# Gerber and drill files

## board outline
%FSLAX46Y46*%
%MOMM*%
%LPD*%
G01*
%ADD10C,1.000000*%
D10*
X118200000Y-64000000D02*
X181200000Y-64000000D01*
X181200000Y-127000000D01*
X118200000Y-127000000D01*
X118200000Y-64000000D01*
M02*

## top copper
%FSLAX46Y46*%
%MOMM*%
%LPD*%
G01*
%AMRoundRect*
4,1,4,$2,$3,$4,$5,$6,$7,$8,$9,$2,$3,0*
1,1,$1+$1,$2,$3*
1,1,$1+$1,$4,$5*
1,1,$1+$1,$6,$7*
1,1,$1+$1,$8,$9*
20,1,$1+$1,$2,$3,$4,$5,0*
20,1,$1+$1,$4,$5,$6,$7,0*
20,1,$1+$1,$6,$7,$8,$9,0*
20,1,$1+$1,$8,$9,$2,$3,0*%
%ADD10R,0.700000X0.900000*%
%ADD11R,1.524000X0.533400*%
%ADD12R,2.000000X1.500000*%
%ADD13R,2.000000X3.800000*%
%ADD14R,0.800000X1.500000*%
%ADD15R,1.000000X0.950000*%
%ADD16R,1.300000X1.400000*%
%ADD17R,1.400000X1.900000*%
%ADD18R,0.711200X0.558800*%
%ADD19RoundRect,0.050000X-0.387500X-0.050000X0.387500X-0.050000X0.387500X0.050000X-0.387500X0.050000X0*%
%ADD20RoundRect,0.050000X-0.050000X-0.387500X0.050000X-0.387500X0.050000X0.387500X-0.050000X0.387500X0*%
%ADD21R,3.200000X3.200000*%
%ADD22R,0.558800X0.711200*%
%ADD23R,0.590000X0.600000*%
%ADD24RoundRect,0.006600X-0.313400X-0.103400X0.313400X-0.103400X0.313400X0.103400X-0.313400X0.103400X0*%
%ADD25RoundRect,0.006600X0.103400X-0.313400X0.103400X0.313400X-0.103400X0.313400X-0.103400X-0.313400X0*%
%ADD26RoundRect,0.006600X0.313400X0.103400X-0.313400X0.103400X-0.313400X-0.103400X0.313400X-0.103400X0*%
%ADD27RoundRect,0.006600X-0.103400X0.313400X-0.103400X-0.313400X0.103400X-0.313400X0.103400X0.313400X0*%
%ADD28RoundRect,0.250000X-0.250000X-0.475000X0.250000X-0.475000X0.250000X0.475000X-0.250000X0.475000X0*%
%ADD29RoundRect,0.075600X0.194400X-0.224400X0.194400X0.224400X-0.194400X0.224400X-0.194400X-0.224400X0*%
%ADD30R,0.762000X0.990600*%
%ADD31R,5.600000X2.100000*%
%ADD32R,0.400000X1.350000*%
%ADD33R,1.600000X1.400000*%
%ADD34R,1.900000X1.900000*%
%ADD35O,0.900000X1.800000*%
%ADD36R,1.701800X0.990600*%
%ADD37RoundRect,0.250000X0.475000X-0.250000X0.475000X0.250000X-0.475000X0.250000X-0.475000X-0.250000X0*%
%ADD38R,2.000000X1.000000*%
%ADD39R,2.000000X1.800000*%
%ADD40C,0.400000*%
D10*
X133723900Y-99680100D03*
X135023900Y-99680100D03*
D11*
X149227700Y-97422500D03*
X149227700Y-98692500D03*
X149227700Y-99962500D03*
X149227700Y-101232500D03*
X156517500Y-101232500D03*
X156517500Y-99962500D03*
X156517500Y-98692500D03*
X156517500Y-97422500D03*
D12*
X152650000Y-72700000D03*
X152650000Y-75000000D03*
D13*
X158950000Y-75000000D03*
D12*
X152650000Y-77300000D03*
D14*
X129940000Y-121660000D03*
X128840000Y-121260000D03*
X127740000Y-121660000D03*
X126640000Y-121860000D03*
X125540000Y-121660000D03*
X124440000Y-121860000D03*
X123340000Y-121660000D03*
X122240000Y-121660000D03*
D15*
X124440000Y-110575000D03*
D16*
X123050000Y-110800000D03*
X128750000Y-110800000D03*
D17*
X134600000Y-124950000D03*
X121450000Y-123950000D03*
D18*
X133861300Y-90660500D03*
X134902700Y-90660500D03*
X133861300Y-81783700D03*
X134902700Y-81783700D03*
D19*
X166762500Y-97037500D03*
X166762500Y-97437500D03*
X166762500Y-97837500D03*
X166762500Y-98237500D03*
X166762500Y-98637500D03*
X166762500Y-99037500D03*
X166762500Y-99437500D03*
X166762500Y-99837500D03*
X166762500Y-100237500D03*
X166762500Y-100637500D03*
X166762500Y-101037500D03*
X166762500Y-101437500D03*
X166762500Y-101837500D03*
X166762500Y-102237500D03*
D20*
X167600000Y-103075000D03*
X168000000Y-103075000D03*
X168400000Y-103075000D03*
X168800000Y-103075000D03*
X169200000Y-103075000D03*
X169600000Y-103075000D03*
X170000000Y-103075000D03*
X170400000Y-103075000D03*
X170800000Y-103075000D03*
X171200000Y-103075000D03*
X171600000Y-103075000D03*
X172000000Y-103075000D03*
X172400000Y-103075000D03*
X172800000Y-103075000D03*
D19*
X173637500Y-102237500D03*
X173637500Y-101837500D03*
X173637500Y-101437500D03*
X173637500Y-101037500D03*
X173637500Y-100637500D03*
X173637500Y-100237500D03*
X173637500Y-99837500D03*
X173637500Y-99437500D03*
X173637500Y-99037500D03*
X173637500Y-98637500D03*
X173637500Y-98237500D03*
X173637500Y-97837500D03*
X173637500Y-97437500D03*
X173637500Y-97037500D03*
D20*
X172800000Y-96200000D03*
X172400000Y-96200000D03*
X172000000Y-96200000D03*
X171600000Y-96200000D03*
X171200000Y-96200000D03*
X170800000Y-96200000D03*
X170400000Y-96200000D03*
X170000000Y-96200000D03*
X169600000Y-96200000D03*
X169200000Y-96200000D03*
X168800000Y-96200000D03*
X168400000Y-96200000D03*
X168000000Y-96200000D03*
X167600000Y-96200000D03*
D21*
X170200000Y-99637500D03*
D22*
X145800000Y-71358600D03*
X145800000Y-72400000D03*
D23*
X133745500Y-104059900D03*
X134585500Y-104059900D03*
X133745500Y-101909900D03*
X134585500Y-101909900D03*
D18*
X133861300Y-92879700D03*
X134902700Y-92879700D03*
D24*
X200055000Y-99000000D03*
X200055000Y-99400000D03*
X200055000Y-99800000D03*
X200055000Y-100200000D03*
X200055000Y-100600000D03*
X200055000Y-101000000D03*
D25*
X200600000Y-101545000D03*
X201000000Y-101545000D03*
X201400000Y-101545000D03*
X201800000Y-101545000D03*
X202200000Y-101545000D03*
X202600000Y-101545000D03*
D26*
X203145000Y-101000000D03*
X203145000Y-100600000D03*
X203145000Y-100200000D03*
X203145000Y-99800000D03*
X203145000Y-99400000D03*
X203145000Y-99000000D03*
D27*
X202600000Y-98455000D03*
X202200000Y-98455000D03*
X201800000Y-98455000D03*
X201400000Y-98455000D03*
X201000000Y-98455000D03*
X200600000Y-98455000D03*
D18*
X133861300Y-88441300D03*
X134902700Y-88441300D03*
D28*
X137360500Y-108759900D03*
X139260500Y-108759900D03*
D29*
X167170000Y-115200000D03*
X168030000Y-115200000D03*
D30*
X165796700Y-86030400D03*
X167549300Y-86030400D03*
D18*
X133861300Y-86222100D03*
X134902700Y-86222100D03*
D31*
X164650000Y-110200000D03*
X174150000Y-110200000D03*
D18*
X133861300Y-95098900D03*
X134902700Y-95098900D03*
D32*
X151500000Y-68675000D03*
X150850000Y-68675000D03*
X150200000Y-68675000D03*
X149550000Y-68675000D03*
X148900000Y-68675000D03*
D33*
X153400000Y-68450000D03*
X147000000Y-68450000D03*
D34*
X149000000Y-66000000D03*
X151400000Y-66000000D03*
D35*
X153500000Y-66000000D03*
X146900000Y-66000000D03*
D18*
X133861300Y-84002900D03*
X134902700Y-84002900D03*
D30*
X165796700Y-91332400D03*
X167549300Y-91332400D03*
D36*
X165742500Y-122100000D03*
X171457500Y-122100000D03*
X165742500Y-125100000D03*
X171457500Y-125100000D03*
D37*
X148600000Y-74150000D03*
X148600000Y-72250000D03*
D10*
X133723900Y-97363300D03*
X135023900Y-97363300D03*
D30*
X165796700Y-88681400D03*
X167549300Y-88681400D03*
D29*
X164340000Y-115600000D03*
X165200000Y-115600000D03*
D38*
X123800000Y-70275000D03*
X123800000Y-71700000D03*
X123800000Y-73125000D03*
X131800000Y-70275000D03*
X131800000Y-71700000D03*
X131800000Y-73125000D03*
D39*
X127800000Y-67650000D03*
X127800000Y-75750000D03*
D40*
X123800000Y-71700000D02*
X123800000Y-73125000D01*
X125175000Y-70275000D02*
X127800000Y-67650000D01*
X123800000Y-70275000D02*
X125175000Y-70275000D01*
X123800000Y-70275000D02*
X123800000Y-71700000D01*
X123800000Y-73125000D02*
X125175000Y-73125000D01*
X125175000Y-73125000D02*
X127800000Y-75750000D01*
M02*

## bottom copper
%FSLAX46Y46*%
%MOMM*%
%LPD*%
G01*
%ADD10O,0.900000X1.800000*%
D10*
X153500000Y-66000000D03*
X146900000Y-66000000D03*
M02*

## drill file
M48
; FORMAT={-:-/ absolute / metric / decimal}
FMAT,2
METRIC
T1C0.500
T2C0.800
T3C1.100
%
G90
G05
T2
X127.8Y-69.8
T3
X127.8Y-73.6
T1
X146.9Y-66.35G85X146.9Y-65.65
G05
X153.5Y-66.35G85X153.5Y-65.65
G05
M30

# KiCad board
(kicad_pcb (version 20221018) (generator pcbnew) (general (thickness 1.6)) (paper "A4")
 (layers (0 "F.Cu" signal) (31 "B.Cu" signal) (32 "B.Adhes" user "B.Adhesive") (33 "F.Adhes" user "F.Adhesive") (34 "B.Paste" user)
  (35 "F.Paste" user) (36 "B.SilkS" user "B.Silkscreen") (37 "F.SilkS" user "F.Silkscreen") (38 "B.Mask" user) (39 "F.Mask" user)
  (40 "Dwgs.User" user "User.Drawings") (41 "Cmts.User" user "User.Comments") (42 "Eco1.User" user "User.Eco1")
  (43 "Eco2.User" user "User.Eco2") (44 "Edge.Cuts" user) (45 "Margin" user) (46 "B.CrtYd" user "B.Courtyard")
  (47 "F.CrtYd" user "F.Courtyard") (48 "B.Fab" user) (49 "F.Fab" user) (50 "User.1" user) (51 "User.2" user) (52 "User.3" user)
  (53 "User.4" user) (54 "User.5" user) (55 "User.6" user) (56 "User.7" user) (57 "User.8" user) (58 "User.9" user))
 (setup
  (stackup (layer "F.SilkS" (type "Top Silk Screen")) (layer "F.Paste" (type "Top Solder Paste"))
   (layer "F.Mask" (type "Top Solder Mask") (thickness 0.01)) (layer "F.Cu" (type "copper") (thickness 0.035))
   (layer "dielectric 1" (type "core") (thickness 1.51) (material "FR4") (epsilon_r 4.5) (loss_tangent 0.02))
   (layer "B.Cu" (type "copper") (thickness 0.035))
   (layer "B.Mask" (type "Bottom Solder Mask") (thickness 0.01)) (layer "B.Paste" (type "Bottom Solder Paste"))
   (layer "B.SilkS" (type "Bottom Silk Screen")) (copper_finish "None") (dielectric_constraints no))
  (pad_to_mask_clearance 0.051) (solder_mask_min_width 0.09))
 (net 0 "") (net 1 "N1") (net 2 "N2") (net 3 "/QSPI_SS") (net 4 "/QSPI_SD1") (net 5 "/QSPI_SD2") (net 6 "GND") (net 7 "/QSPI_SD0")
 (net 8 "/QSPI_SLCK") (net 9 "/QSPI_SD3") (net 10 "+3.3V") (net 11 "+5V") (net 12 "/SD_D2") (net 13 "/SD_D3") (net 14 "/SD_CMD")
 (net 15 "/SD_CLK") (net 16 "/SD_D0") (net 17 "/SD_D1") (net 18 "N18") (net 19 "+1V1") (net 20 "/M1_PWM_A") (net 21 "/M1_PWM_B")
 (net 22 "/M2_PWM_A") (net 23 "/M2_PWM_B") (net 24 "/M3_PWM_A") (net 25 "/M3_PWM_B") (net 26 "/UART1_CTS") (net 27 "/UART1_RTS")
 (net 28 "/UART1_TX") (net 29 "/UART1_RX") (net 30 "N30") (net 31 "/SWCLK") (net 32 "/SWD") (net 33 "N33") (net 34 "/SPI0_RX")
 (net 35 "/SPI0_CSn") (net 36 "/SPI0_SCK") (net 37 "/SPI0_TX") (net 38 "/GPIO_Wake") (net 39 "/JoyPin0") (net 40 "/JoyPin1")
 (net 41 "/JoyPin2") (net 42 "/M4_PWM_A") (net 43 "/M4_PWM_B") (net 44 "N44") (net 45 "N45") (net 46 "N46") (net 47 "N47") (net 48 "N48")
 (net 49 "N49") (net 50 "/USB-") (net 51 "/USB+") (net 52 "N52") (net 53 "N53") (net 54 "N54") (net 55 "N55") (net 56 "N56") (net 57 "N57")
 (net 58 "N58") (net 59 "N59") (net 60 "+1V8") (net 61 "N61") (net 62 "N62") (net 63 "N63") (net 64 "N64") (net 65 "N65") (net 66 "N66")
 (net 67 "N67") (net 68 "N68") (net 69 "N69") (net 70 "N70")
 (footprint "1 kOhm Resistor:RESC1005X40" (layer "F.Cu") (at 134.3739 99.6801)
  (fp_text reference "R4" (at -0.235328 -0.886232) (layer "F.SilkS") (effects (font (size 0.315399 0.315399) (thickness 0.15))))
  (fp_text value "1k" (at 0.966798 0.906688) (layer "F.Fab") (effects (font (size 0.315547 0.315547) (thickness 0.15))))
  (pad "1" smd rect (at -0.65 0) (size 0.7 0.9) (layers "F.Cu" "F.Paste" "F.Mask") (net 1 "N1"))
  (pad "2" smd rect (at 0.65 0) (size 0.7 0.9) (layers "F.Cu" "F.Paste" "F.Mask") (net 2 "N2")))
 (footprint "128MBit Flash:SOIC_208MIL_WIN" (layer "F.Cu") (at 152.8726 99.3275)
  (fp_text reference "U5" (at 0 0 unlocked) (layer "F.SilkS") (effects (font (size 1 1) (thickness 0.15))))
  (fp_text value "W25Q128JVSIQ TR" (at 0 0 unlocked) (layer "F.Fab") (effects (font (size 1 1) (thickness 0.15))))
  (pad "1" smd rect (at -3.6449 -1.905) (size 1.524 0.5334) (layers "F.Cu" "F.Paste" "F.Mask") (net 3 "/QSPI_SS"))
  (pad "2" smd rect (at -3.6449 -0.635) (size 1.524 0.5334) (layers "F.Cu" "F.Paste" "F.Mask") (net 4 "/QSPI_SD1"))
  (pad "3" smd rect (at -3.6449 0.635) (size 1.524 0.5334) (layers "F.Cu" "F.Paste" "F.Mask") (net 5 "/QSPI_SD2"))
  (pad "4" smd rect (at -3.6449 1.905) (size 1.524 0.5334) (layers "F.Cu" "F.Paste" "F.Mask") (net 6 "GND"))
  (pad "5" smd rect (at 3.6449 1.905) (size 1.524 0.5334) (layers "F.Cu" "F.Paste" "F.Mask") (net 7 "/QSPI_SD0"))
  (pad "6" smd rect (at 3.6449 0.635) (size 1.524 0.5334) (layers "F.Cu" "F.Paste" "F.Mask") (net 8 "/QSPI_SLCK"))
  (pad "7" smd rect (at 3.6449 -0.635) (size 1.524 0.5334) (layers "F.Cu" "F.Paste" "F.Mask") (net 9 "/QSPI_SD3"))
  (pad "8" smd rect (at 3.6449 -1.905) (size 1.524 0.5334) (layers "F.Cu" "F.Paste" "F.Mask") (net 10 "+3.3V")))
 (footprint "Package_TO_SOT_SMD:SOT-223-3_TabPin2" (layer "F.Cu") (at 155.8 75)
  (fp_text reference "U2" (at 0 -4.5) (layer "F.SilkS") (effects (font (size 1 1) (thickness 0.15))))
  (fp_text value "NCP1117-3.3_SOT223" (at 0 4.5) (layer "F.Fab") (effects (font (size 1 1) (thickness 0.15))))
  (pad "1" smd rect (at -3.15 -2.3) (size 2 1.5) (layers "F.Cu" "F.Paste" "F.Mask") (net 6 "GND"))
  (pad "2" smd rect (at -3.15 0) (size 2 1.5) (layers "F.Cu" "F.Paste" "F.Mask") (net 10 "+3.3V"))
  (pad "2" smd rect (at 3.15 0) (size 2 3.8) (layers "F.Cu" "F.Paste" "F.Mask") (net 10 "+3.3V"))
  (pad "3" smd rect (at -3.15 2.3) (size 2 1.5) (layers "F.Cu" "F.Paste" "F.Mask") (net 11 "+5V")))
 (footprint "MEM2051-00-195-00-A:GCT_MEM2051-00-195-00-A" (layer "F.Cu") (at 128 118)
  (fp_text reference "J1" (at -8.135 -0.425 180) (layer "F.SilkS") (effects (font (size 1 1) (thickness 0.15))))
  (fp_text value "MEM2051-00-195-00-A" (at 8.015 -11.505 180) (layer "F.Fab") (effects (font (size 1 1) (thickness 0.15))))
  (pad "1" smd rect (at 1.94 3.66) (size 0.8 1.5) (layers "F.Cu" "F.Paste" "F.Mask") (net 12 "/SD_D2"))
  (pad "2" smd rect (at 0.84 3.26) (size 0.8 1.5) (layers "F.Cu" "F.Paste" "F.Mask") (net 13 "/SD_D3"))
  (pad "3" smd rect (at -0.26 3.66) (size 0.8 1.5) (layers "F.Cu" "F.Paste" "F.Mask") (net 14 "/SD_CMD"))
  (pad "4" smd rect (at -1.36 3.86) (size 0.8 1.5) (layers "F.Cu" "F.Paste" "F.Mask") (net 10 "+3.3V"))
  (pad "5" smd rect (at -2.46 3.66) (size 0.8 1.5) (layers "F.Cu" "F.Paste" "F.Mask") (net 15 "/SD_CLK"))
  (pad "6" smd rect (at -3.56 3.86) (size 0.8 1.5) (layers "F.Cu" "F.Paste" "F.Mask") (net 6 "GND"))
  (pad "7" smd rect (at -4.66 3.66) (size 0.8 1.5) (layers "F.Cu" "F.Paste" "F.Mask") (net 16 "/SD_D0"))
  (pad "8" smd rect (at -5.76 3.66) (size 0.8 1.5) (layers "F.Cu" "F.Paste" "F.Mask") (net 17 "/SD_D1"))
  (pad "9" smd rect (at -3.56 -7.425) (size 1 0.95) (layers "F.Cu" "F.Paste" "F.Mask") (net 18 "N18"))
  (pad "P1" smd rect (at -4.95 -7.2) (size 1.3 1.4) (layers "F.Cu" "F.Paste" "F.Mask"))
  (pad "P2" smd rect (at 0.75 -7.2) (size 1.3 1.4) (layers "F.Cu" "F.Paste" "F.Mask"))
  (pad "P3" smd rect (at 6.6 6.95) (size 1.4 1.9) (layers "F.Cu" "F.Paste" "F.Mask"))
  (pad "P4" smd rect (at -6.55 5.95) (size 1.4 1.9) (layers "F.Cu" "F.Paste" "F.Mask")))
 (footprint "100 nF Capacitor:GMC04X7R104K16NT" (layer "F.Cu") (at 134.382 90.6605)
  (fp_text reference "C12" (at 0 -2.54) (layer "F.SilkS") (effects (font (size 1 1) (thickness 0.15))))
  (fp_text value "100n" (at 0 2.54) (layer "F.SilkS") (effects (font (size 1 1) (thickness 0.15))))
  (pad "1" smd rect (at -0.5207 0) (size 0.7112 0.5588) (layers "F.Cu" "F.Paste" "F.Mask") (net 6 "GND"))
  (pad "2" smd rect (at 0.5207 0) (size 0.7112 0.5588) (layers "F.Cu" "F.Paste" "F.Mask") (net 10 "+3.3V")))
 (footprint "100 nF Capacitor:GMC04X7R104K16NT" (layer "F.Cu") (at 134.382 81.7837)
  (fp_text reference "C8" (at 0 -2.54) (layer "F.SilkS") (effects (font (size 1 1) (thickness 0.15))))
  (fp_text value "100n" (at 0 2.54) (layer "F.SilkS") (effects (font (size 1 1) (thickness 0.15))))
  (pad "1" smd rect (at -0.5207 0) (size 0.7112 0.5588) (layers "F.Cu" "F.Paste" "F.Mask") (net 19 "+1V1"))
  (pad "2" smd rect (at 0.5207 0) (size 0.7112 0.5588) (layers "F.Cu" "F.Paste" "F.Mask") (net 6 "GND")))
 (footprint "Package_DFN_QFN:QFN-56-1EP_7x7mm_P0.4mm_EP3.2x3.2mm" (layer "F.Cu") (at 170.2 99.6375)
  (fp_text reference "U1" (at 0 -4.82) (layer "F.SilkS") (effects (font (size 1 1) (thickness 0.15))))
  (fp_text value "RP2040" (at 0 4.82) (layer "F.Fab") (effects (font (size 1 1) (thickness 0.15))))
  (pad "" smd roundrect (at -0.8 -0.8) (size 1.29 1.29) (layers "F.Paste") (roundrect_rratio 0.193798))
  (pad "" smd roundrect (at -0.8 0.8) (size 1.29 1.29) (layers "F.Paste") (roundrect_rratio 0.193798))
  (pad "" smd roundrect (at 0.8 -0.8) (size 1.29 1.29) (layers "F.Paste") (roundrect_rratio 0.193798))
  (pad "" smd roundrect (at 0.8 0.8) (size 1.29 1.29) (layers "F.Paste") (roundrect_rratio 0.193798))
  (pad "1" smd roundrect (at -3.4375 -2.6) (size 0.875 0.2) (layers "F.Cu" "F.Paste" "F.Mask") (roundrect_rratio 0.25) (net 10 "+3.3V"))
  (pad "2" smd roundrect (at -3.4375 -2.2) (size 0.875 0.2) (layers "F.Cu" "F.Paste" "F.Mask") (roundrect_rratio 0.25) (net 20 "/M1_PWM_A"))
  (pad "3" smd roundrect (at -3.4375 -1.8) (size 0.875 0.2) (layers "F.Cu" "F.Paste" "F.Mask") (roundrect_rratio 0.25) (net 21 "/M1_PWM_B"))
  (pad "4" smd roundrect (at -3.4375 -1.4) (size 0.875 0.2) (layers "F.Cu" "F.Paste" "F.Mask") (roundrect_rratio 0.25) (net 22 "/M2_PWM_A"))
  (pad "5" smd roundrect (at -3.4375 -1) (size 0.875 0.2) (layers "F.Cu" "F.Paste" "F.Mask") (roundrect_rratio 0.25) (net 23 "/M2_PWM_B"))
  (pad "6" smd roundrect (at -3.4375 -0.6) (size 0.875 0.2) (layers "F.Cu" "F.Paste" "F.Mask") (roundrect_rratio 0.25) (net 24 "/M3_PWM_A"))
  (pad "7" smd roundrect (at -3.4375 -0.2) (size 0.875 0.2) (layers "F.Cu" "F.Paste" "F.Mask") (roundrect_rratio 0.25) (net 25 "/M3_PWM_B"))
  (pad "8" smd roundrect (at -3.4375 0.2) (size 0.875 0.2) (layers "F.Cu" "F.Paste" "F.Mask") (roundrect_rratio 0.25) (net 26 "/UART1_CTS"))
  (pad "9" smd roundrect (at -3.4375 0.6) (size 0.875 0.2) (layers "F.Cu" "F.Paste" "F.Mask") (roundrect_rratio 0.25) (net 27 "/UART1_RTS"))
  (pad "10" smd roundrect (at -3.4375 1) (size 0.875 0.2) (layers "F.Cu" "F.Paste" "F.Mask") (roundrect_rratio 0.25) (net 10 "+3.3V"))
  (pad "11" smd roundrect (at -3.4375 1.4) (size 0.875 0.2) (layers "F.Cu" "F.Paste" "F.Mask") (roundrect_rratio 0.25) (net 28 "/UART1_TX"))
  (pad "12" smd roundrect (at -3.4375 1.8) (size 0.875 0.2) (layers "F.Cu" "F.Paste" "F.Mask") (roundrect_rratio 0.25) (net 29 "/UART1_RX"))
  (pad "13" smd roundrect (at -3.4375 2.2) (size 0.875 0.2) (layers "F.Cu" "F.Paste" "F.Mask") (roundrect_rratio 0.25) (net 14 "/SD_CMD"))
  (pad "14" smd roundrect (at -3.4375 2.6) (size 0.875 0.2) (layers "F.Cu" "F.Paste" "F.Mask") (roundrect_rratio 0.25) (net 15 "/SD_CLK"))
  (pad "15" smd roundrect (at -2.6 3.4375) (size 0.2 0.875) (layers "F.Cu" "F.Paste" "F.Mask") (roundrect_rratio 0.25) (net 16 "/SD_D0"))
  (pad "16" smd roundrect (at -2.2 3.4375) (size 0.2 0.875) (layers "F.Cu" "F.Paste" "F.Mask") (roundrect_rratio 0.25) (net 17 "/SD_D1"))
  (pad "17" smd roundrect (at -1.8 3.4375) (size 0.2 0.875) (layers "F.Cu" "F.Paste" "F.Mask") (roundrect_rratio 0.25) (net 12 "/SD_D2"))
  (pad "18" smd roundrect (at -1.4 3.4375) (size 0.2 0.875) (layers "F.Cu" "F.Paste" "F.Mask") (roundrect_rratio 0.25) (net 13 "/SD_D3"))
  (pad "19" smd roundrect (at -1 3.4375) (size 0.2 0.875) (layers "F.Cu" "F.Paste" "F.Mask") (roundrect_rratio 0.25) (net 6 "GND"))
  (pad "20" smd roundrect (at -0.6 3.4375) (size 0.2 0.875) (layers "F.Cu" "F.Paste" "F.Mask") (roundrect_rratio 0.25) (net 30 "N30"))
  (pad "21" smd roundrect (at -0.2 3.4375) (size 0.2 0.875) (layers "F.Cu" "F.Paste" "F.Mask") (roundrect_rratio 0.25) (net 1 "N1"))
  (pad "22" smd roundrect (at 0.2 3.4375) (size 0.2 0.875) (layers "F.Cu" "F.Paste" "F.Mask") (roundrect_rratio 0.25) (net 10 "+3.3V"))
  (pad "23" smd roundrect (at 0.6 3.4375) (size 0.2 0.875) (layers "F.Cu" "F.Paste" "F.Mask") (roundrect_rratio 0.25) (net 19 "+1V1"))
  (pad "24" smd roundrect (at 1 3.4375) (size 0.2 0.875) (layers "F.Cu" "F.Paste" "F.Mask") (roundrect_rratio 0.25) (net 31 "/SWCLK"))
  (pad "25" smd roundrect (at 1.4 3.4375) (size 0.2 0.875) (layers "F.Cu" "F.Paste" "F.Mask") (roundrect_rratio 0.25) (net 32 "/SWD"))
  (pad "26" smd roundrect (at 1.8 3.4375) (size 0.2 0.875) (layers "F.Cu" "F.Paste" "F.Mask") (roundrect_rratio 0.25) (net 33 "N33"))
  (pad "27" smd roundrect (at 2.2 3.4375) (size 0.2 0.875) (layers "F.Cu" "F.Paste" "F.Mask") (roundrect_rratio 0.25) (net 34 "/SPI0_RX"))
  (pad "28" smd roundrect (at 2.6 3.4375) (size 0.2 0.875) (layers "F.Cu" "F.Paste" "F.Mask") (roundrect_rratio 0.25) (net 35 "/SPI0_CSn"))
  (pad "29" smd roundrect (at 3.4375 2.6) (size 0.875 0.2) (layers "F.Cu" "F.Paste" "F.Mask") (roundrect_rratio 0.25) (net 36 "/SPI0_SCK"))
  (pad "30" smd roundrect (at 3.4375 2.2) (size 0.875 0.2) (layers "F.Cu" "F.Paste" "F.Mask") (roundrect_rratio 0.25) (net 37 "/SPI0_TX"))
  (pad "31" smd roundrect (at 3.4375 1.8) (size 0.875 0.2) (layers "F.Cu" "F.Paste" "F.Mask") (roundrect_rratio 0.25) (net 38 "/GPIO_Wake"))
  (pad "32" smd roundrect (at 3.4375 1.4) (size 0.875 0.2) (layers "F.Cu" "F.Paste" "F.Mask") (roundrect_rratio 0.25) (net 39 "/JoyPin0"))
  (pad "33" smd roundrect (at 3.4375 1) (size 0.875 0.2) (layers "F.Cu" "F.Paste" "F.Mask") (roundrect_rratio 0.25) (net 10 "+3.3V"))
  (pad "34" smd roundrect (at 3.4375 0.6) (size 0.875 0.2) (layers "F.Cu" "F.Paste" "F.Mask") (roundrect_rratio 0.25) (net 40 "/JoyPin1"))
  (pad "35" smd roundrect (at 3.4375 0.2) (size 0.875 0.2) (layers "F.Cu" "F.Paste" "F.Mask") (roundrect_rratio 0.25) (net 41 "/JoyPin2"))
  (pad "36" smd roundrect (at 3.4375 -0.2) (size 0.875 0.2) (layers "F.Cu" "F.Paste" "F.Mask") (roundrect_rratio 0.25) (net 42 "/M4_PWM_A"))
  (pad "37" smd roundrect (at 3.4375 -0.6) (size 0.875 0.2) (layers "F.Cu" "F.Paste" "F.Mask") (roundrect_rratio 0.25) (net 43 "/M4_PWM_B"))
  (pad "38" smd roundrect (at 3.4375 -1) (size 0.875 0.2) (layers "F.Cu" "F.Paste" "F.Mask") (roundrect_rratio 0.25) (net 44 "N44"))
  (pad "39" smd roundrect (at 3.4375 -1.4) (size 0.875 0.2) (layers "F.Cu" "F.Paste" "F.Mask") (roundrect_rratio 0.25) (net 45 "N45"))
  (pad "40" smd roundrect (at 3.4375 -1.8) (size 0.875 0.2) (layers "F.Cu" "F.Paste" "F.Mask") (roundrect_rratio 0.25) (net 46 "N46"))
  (pad "41" smd roundrect (at 3.4375 -2.2) (size 0.875 0.2) (layers "F.Cu" "F.Paste" "F.Mask") (roundrect_rratio 0.25) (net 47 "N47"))
  (pad "42" smd roundrect (at 3.4375 -2.6) (size 0.875 0.2) (layers "F.Cu" "F.Paste" "F.Mask") (roundrect_rratio 0.25) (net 10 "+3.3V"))
  (pad "43" smd roundrect (at 2.6 -3.4375) (size 0.2 0.875) (layers "F.Cu" "F.Paste" "F.Mask") (roundrect_rratio 0.25) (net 10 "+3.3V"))
  (pad "44" smd roundrect (at 2.2 -3.4375) (size 0.2 0.875) (layers "F.Cu" "F.Paste" "F.Mask") (roundrect_rratio 0.25) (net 10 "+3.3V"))
  (pad "45" smd roundrect (at 1.8 -3.4375) (size 0.2 0.875) (layers "F.Cu" "F.Paste" "F.Mask") (roundrect_rratio 0.25) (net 19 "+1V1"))
  (pad "46" smd roundrect (at 1.4 -3.4375) (size 0.2 0.875) (layers "F.Cu" "F.Paste" "F.Mask") (roundrect_rratio 0.25) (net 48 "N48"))
  (pad "47" smd roundrect (at 1 -3.4375) (size 0.2 0.875) (layers "F.Cu" "F.Paste" "F.Mask") (roundrect_rratio 0.25) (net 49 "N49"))
  (pad "48" smd roundrect (at 0.6 -3.4375) (size 0.2 0.875) (layers "F.Cu" "F.Paste" "F.Mask") (roundrect_rratio 0.25) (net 10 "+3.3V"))
  (pad "49" smd roundrect (at 0.2 -3.4375) (size 0.2 0.875) (layers "F.Cu" "F.Paste" "F.Mask") (roundrect_rratio 0.25) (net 10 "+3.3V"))
  (pad "50" smd roundrect (at -0.2 -3.4375) (size 0.2 0.875) (layers "F.Cu" "F.Paste" "F.Mask") (roundrect_rratio 0.25) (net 19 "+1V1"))
  (pad "51" smd roundrect (at -0.6 -3.4375) (size 0.2 0.875) (layers "F.Cu" "F.Paste" "F.Mask") (roundrect_rratio 0.25) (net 9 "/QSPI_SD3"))
  (pad "52" smd roundrect (at -1 -3.4375) (size 0.2 0.875) (layers "F.Cu" "F.Paste" "F.Mask") (roundrect_rratio 0.25) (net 8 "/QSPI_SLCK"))
  (pad "53" smd roundrect (at -1.4 -3.4375) (size 0.2 0.875) (layers "F.Cu" "F.Paste" "F.Mask") (roundrect_rratio 0.25) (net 7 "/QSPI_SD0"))
  (pad "54" smd roundrect (at -1.8 -3.4375) (size 0.2 0.875) (layers "F.Cu" "F.Paste" "F.Mask") (roundrect_rratio 0.25) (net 5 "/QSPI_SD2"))
  (pad "55" smd roundrect (at -2.2 -3.4375) (size 0.2 0.875) (layers "F.Cu" "F.Paste" "F.Mask") (roundrect_rratio 0.25) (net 4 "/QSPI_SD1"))
  (pad "56" smd roundrect (at -2.6 -3.4375) (size 0.2 0.875) (layers "F.Cu" "F.Paste" "F.Mask") (roundrect_rratio 0.25) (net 3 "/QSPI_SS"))
  (pad "57" smd rect (at 0 0) (size 3.2 3.2) (layers "F.Cu" "F.Mask") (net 6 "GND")))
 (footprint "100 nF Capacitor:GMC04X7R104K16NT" (layer "F.Cu") (at 145.8 71.8793 -90)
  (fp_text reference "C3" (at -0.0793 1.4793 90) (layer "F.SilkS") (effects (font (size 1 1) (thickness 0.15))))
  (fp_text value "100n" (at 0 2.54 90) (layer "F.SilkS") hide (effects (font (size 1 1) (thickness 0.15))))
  (pad "1" smd rect (at -0.5207 0 270) (size 0.7112 0.5588) (layers "F.Cu" "F.Paste" "F.Mask") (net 6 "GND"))
  (pad "2" smd rect (at 0.5207 0 270) (size 0.7112 0.5588) (layers "F.Cu" "F.Paste" "F.Mask") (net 10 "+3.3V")))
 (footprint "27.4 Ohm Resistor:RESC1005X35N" (layer "F.Cu") (at 134.1655 104.0599)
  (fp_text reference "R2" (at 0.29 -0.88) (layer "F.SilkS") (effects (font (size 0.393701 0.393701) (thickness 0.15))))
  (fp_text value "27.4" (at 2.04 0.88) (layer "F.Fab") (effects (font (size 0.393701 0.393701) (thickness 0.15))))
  (pad "1" smd rect (at -0.42 0) (size 0.59 0.6) (layers "F.Cu" "F.Paste" "F.Mask") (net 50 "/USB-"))
  (pad "2" smd rect (at 0.42 0) (size 0.59 0.6) (layers "F.Cu" "F.Paste" "F.Mask") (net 48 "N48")))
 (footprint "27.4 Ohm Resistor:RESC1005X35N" (layer "F.Cu") (at 134.1655 101.9099)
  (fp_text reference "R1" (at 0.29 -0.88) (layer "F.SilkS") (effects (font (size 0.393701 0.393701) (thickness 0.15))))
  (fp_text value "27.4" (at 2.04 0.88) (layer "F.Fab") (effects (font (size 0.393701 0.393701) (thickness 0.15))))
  (pad "1" smd rect (at -0.42 0) (size 0.59 0.6) (layers "F.Cu" "F.Paste" "F.Mask") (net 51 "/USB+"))
  (pad "2" smd rect (at 0.42 0) (size 0.59 0.6) (layers "F.Cu" "F.Paste" "F.Mask") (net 49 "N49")))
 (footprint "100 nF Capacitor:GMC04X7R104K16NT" (layer "F.Cu") (at 134.382 92.8797)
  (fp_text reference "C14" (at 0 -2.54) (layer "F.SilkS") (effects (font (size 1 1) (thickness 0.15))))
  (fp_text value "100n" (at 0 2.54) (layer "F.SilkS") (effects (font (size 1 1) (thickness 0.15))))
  (pad "1" smd rect (at -0.5207 0) (size 0.7112 0.5588) (layers "F.Cu" "F.Paste" "F.Mask") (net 6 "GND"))
  (pad "2" smd rect (at 0.5207 0) (size 0.7112 0.5588) (layers "F.Cu" "F.Paste" "F.Mask") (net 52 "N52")))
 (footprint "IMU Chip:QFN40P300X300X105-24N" (layer "F.Cu") (at 201.6 100)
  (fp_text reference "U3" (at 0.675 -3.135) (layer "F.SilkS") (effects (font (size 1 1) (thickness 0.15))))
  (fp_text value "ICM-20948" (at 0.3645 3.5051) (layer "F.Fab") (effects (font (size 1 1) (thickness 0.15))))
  (pad "1" smd roundrect (at -1.545 -1) (size 0.64 0.22) (layers "F.Cu" "F.Paste" "F.Mask") (roundrect_rratio 0.03) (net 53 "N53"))
  (pad "2" smd roundrect (at -1.545 -0.6) (size 0.64 0.22) (layers "F.Cu" "F.Paste" "F.Mask") (roundrect_rratio 0.03) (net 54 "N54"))
  (pad "3" smd roundrect (at -1.545 -0.2) (size 0.64 0.22) (layers "F.Cu" "F.Paste" "F.Mask") (roundrect_rratio 0.03) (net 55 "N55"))
  (pad "4" smd roundrect (at -1.545 0.2) (size 0.64 0.22) (layers "F.Cu" "F.Paste" "F.Mask") (roundrect_rratio 0.03) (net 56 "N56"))
  (pad "5" smd roundrect (at -1.545 0.6) (size 0.64 0.22) (layers "F.Cu" "F.Paste" "F.Mask") (roundrect_rratio 0.03) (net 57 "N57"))
  (pad "6" smd roundrect (at -1.545 1) (size 0.64 0.22) (layers "F.Cu" "F.Paste" "F.Mask") (roundrect_rratio 0.03) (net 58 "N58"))
  (pad "7" smd roundrect (at -1 1.545 90) (size 0.64 0.22) (layers "F.Cu" "F.Paste" "F.Mask") (roundrect_rratio 0.03) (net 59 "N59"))
  (pad "8" smd roundrect (at -0.6 1.545 90) (size 0.64 0.22) (layers "F.Cu" "F.Paste" "F.Mask") (roundrect_rratio 0.03) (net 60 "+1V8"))
  (pad "9" smd roundrect (at -0.2 1.545 90) (size 0.64 0.22) (layers "F.Cu" "F.Paste" "F.Mask") (roundrect_rratio 0.03) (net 34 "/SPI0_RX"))
  (pad "10" smd roundrect (at 0.2 1.545 90) (size 0.64 0.22) (layers "F.Cu" "F.Paste" "F.Mask") (roundrect_rratio 0.03) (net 52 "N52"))
  (pad "11" smd roundrect (at 0.6 1.545 90) (size 0.64 0.22) (layers "F.Cu" "F.Paste" "F.Mask") (roundrect_rratio 0.03) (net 6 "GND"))
  (pad "12" smd roundrect (at 1 1.545 90) (size 0.64 0.22) (layers "F.Cu" "F.Paste" "F.Mask") (roundrect_rratio 0.03) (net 38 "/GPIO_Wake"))
  (pad "13" smd roundrect (at 1.545 1 180) (size 0.64 0.22) (layers "F.Cu" "F.Paste" "F.Mask") (roundrect_rratio 0.03) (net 10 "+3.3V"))
  (pad "14" smd roundrect (at 1.545 0.6 180) (size 0.64 0.22) (layers "F.Cu" "F.Paste" "F.Mask") (roundrect_rratio 0.03) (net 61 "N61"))
  (pad "15" smd roundrect (at 1.545 0.2 180) (size 0.64 0.22) (layers "F.Cu" "F.Paste" "F.Mask") (roundrect_rratio 0.03) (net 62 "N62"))
  (pad "16" smd roundrect (at 1.545 -0.2 180) (size 0.64 0.22) (layers "F.Cu" "F.Paste" "F.Mask") (roundrect_rratio 0.03) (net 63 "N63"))
  (pad "17" smd roundrect (at 1.545 -0.6 180) (size 0.64 0.22) (layers "F.Cu" "F.Paste" "F.Mask") (roundrect_rratio 0.03) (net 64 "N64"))
  (pad "18" smd roundrect (at 1.545 -1 180) (size 0.64 0.22) (layers "F.Cu" "F.Paste" "F.Mask") (roundrect_rratio 0.03) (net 6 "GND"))
  (pad "19" smd roundrect (at 1 -1.545 270) (size 0.64 0.22) (layers "F.Cu" "F.Paste" "F.Mask") (roundrect_rratio 0.03) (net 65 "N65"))
  (pad "20" smd roundrect (at 0.6 -1.545 270) (size 0.64 0.22) (layers "F.Cu" "F.Paste" "F.Mask") (roundrect_rratio 0.03) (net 6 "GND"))
  (pad "21" smd roundrect (at 0.2 -1.545 270) (size 0.64 0.22) (layers "F.Cu" "F.Paste" "F.Mask") (roundrect_rratio 0.03) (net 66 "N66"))
  (pad "22" smd roundrect (at -0.2 -1.545 270) (size 0.64 0.22) (layers "F.Cu" "F.Paste" "F.Mask") (roundrect_rratio 0.03)
   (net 35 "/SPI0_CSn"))
  (pad "23" smd roundrect (at -0.6 -1.545 270) (size 0.64 0.22) (layers "F.Cu" "F.Paste" "F.Mask") (roundrect_rratio 0.03)
   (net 36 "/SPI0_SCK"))
  (pad "24" smd roundrect (at -1 -1.545 270) (size 0.64 0.22) (layers "F.Cu" "F.Paste" "F.Mask") (roundrect_rratio 0.03) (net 37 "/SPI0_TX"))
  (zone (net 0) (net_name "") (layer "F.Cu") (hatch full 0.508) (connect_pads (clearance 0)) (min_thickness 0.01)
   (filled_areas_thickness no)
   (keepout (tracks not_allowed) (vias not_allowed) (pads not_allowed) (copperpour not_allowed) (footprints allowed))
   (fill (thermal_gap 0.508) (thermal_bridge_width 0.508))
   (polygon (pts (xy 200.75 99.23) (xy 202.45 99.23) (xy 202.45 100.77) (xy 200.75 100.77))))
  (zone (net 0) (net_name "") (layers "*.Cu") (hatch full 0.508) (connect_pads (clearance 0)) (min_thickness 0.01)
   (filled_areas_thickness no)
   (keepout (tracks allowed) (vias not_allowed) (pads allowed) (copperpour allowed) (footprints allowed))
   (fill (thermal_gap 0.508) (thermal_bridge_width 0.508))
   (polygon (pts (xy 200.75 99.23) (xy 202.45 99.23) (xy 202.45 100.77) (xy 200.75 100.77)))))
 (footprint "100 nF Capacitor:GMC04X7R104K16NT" (layer "F.Cu") (at 134.382 88.4413)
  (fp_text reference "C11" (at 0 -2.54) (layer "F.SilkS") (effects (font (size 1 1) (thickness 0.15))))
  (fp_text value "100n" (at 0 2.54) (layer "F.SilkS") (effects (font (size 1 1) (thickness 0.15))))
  (pad "1" smd rect (at -0.5207 0) (size 0.7112 0.5588) (layers "F.Cu" "F.Paste" "F.Mask") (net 10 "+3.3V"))
  (pad "2" smd rect (at 0.5207 0) (size 0.7112 0.5588) (layers "F.Cu" "F.Paste" "F.Mask") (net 6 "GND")))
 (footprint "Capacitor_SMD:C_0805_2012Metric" (layer "F.Cu") (at 138.3105 108.7599)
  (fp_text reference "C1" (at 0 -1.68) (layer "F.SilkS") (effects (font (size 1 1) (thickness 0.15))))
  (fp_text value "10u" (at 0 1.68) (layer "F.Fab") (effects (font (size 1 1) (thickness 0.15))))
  (pad "1" smd roundrect (at -0.95 0) (size 1 1.45) (layers "F.Cu" "F.Paste" "F.Mask") (roundrect_rratio 0.25) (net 11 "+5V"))
  (pad "2" smd roundrect (at 0.95 0) (size 1 1.45) (layers "F.Cu" "F.Paste" "F.Mask") (roundrect_rratio 0.25) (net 6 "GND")))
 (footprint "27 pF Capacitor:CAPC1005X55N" (layer "F.Cu") (at 167.6 115.2)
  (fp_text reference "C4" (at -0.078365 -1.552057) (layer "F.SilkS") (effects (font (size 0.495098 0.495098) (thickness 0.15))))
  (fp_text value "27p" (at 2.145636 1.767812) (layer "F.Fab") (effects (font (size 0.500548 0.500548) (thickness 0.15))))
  (pad "1" smd roundrect (at -0.43 0 90) (size 0.6 0.54) (layers "F.Cu" "F.Paste" "F.Mask") (roundrect_rratio 0.14) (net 30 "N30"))
  (pad "2" smd roundrect (at 0.43 0 90) (size 0.6 0.54) (layers "F.Cu" "F.Paste" "F.Mask") (roundrect_rratio 0.14) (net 6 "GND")))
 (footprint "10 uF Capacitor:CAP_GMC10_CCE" (layer "F.Cu") (at 166.673 86.0304)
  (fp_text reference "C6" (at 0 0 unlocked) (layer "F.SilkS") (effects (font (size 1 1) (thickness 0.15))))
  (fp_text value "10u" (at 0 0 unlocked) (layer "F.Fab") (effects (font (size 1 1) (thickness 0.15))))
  (pad "1" smd rect (at -0.8763 0) (size 0.762 0.9906) (layers "F.Cu" "F.Paste" "F.Mask") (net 6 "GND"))
  (pad "2" smd rect (at 0.8763 0) (size 0.762 0.9906) (layers "F.Cu" "F.Paste" "F.Mask") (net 10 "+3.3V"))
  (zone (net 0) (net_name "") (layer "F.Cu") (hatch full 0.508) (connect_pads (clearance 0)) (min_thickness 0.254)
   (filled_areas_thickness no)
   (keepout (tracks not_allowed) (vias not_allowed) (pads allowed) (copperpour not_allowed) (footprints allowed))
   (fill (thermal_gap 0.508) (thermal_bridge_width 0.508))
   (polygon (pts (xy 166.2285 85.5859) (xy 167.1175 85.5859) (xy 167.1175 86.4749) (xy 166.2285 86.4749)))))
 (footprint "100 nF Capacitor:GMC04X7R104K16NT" (layer "F.Cu") (at 134.382 86.2221)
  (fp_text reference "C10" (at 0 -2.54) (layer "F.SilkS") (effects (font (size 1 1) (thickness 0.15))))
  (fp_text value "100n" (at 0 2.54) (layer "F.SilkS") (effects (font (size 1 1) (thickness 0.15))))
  (pad "1" smd rect (at -0.5207 0) (size 0.7112 0.5588) (layers "F.Cu" "F.Paste" "F.Mask") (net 10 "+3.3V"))
  (pad "2" smd rect (at 0.5207 0) (size 0.7112 0.5588) (layers "F.Cu" "F.Paste" "F.Mask") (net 6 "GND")))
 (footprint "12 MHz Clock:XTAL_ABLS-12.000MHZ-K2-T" (layer "F.Cu") (at 169.4 110.2)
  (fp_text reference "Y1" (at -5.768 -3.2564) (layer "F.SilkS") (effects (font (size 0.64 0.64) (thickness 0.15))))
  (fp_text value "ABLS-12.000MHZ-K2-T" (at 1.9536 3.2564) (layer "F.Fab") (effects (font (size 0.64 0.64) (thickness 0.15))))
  (pad "1" smd rect (at -4.75 0) (size 5.6 2.1) (layers "F.Cu" "F.Paste" "F.Mask") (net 2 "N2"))
  (pad "2" smd rect (at 4.75 0) (size 5.6 2.1) (layers "F.Cu" "F.Paste" "F.Mask") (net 30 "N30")))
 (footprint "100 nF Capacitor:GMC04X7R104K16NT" (layer "F.Cu") (at 134.382 95.0989)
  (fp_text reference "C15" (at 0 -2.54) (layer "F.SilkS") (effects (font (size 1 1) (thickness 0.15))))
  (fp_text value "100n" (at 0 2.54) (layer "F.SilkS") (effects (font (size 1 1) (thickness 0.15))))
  (pad "1" smd rect (at -0.5207 0) (size 0.7112 0.5588) (layers "F.Cu" "F.Paste" "F.Mask") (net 6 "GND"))
  (pad "2" smd rect (at 0.5207 0) (size 0.7112 0.5588) (layers "F.Cu" "F.Paste" "F.Mask") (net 60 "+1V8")))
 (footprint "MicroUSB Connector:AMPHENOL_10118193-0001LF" (layer "F.Cu") (at 150.2 66 180)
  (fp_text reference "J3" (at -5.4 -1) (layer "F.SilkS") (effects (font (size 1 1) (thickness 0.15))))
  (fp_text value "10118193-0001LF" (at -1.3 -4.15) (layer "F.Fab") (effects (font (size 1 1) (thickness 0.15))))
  (pad "1" smd rect (at -1.3 -2.675 180) (size 0.4 1.35) (layers "F.Cu" "F.Paste" "F.Mask") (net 11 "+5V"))
  (pad "2" smd rect (at -0.65 -2.675 180) (size 0.4 1.35) (layers "F.Cu" "F.Paste" "F.Mask") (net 50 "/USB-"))
  (pad "3" smd rect (at 0 -2.675 180) (size 0.4 1.35) (layers "F.Cu" "F.Paste" "F.Mask") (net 51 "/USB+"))
  (pad "4" smd rect (at 0.65 -2.675 180) (size 0.4 1.35) (layers "F.Cu" "F.Paste" "F.Mask") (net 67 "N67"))
  (pad "5" smd rect (at 1.3 -2.675 180) (size 0.4 1.35) (layers "F.Cu" "F.Paste" "F.Mask") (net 6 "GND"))
  (pad "S1" smd rect (at -3.2 -2.45 180) (size 1.6 1.4) (layers "F.Cu" "F.Paste" "F.Mask") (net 6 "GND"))
  (pad "S2" smd rect (at 3.2 -2.45 180) (size 1.6 1.4) (layers "F.Cu" "F.Paste" "F.Mask") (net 6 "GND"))
  (pad "S3" smd rect (at 1.2 0 180) (size 1.9 1.9) (layers "F.Cu" "F.Paste" "F.Mask") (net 6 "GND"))
  (pad "S4" smd rect (at -1.2 0 180) (size 1.9 1.9) (layers "F.Cu" "F.Paste" "F.Mask") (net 6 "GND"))
  (pad "S5" thru_hole oval (at -3.3 0 180) (size 0.9 1.8) (drill oval 0.5 1.2) (layers "*.Cu" "*.Mask") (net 6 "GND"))
  (pad "S6" thru_hole oval (at 3.3 0 180) (size 0.9 1.8) (drill oval 0.5 1.2) (layers "*.Cu" "*.Mask") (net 6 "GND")))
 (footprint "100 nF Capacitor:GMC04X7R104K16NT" (layer "F.Cu") (at 134.382 84.0029)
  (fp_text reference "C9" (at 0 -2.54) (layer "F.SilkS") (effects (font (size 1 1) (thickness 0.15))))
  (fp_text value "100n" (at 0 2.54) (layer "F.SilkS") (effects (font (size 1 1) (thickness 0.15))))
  (pad "1" smd rect (at -0.5207 0) (size 0.7112 0.5588) (layers "F.Cu" "F.Paste" "F.Mask") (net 10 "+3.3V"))
  (pad "2" smd rect (at 0.5207 0) (size 0.7112 0.5588) (layers "F.Cu" "F.Paste" "F.Mask") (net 6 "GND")))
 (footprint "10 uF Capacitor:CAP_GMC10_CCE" (layer "F.Cu") (at 166.673 91.3324)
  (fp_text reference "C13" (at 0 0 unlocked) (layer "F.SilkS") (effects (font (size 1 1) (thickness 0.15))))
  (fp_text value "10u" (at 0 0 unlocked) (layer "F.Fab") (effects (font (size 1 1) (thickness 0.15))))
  (pad "1" smd rect (at -0.8763 0) (size 0.762 0.9906) (layers "F.Cu" "F.Paste" "F.Mask"))
  (pad "2" smd rect (at 0.8763 0) (size 0.762 0.9906) (layers "F.Cu" "F.Paste" "F.Mask"))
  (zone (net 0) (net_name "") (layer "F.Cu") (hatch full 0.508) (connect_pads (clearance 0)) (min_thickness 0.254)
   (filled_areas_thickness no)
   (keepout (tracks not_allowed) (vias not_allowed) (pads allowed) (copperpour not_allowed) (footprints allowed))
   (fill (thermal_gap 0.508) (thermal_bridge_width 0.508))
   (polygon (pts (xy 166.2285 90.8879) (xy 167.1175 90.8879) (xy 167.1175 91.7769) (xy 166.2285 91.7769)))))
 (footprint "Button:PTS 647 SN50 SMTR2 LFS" (layer "F.Cu") (at 168.6 123.6)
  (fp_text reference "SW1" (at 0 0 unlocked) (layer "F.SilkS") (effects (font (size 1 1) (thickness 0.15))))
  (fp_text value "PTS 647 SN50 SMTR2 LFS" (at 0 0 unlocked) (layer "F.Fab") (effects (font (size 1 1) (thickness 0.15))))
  (pad "1" smd rect (at -2.8575 -1.5) (size 1.7018 0.9906) (layers "F.Cu" "F.Paste" "F.Mask") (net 6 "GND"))
  (pad "2" smd rect (at 2.8575 -1.5) (size 1.7018 0.9906) (layers "F.Cu" "F.Paste" "F.Mask") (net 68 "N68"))
  (pad "3" smd rect (at -2.8575 1.5) (size 1.7018 0.9906) (layers "F.Cu" "F.Paste" "F.Mask") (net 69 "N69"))
  (pad "4" smd rect (at 2.8575 1.5) (size 1.7018 0.9906) (layers "F.Cu" "F.Paste" "F.Mask") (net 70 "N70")))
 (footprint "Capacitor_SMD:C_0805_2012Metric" (layer "F.Cu") (at 148.6 73.2 90)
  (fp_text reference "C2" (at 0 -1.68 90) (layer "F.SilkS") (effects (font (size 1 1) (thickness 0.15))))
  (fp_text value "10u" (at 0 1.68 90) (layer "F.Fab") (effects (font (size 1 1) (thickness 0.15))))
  (pad "1" smd roundrect (at -0.95 0 90) (size 1 1.45) (layers "F.Cu" "F.Paste" "F.Mask") (roundrect_rratio 0.25) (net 10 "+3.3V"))
  (pad "2" smd roundrect (at 0.95 0 90) (size 1 1.45) (layers "F.Cu" "F.Paste" "F.Mask") (roundrect_rratio 0.25) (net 6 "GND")))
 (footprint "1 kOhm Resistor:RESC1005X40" (layer "F.Cu") (at 134.3739 97.3633)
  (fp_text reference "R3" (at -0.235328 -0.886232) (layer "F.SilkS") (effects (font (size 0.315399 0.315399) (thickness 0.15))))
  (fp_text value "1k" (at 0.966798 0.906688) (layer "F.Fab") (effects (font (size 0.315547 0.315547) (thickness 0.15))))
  (pad "1" smd rect (at -0.65 0) (size 0.7 0.9) (layers "F.Cu" "F.Paste" "F.Mask") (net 3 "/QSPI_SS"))
  (pad "2" smd rect (at 0.65 0) (size 0.7 0.9) (layers "F.Cu" "F.Paste" "F.Mask") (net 70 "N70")))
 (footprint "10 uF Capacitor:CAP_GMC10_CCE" (layer "F.Cu") (at 166.673 88.6814)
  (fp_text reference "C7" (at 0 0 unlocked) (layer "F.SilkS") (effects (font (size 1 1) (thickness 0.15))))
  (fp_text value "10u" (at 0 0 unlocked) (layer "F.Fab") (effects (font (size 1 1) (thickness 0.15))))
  (pad "1" smd rect (at -0.8763 0) (size 0.762 0.9906) (layers "F.Cu" "F.Paste" "F.Mask") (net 6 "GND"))
  (pad "2" smd rect (at 0.8763 0) (size 0.762 0.9906) (layers "F.Cu" "F.Paste" "F.Mask") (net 19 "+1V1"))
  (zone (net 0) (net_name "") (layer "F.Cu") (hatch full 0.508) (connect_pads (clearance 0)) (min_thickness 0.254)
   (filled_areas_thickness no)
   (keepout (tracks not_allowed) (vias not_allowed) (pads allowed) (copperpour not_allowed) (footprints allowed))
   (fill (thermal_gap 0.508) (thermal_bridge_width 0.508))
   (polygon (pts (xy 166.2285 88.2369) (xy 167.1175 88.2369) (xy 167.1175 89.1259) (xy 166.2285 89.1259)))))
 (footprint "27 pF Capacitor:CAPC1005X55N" (layer "F.Cu") (at 164.77 115.6)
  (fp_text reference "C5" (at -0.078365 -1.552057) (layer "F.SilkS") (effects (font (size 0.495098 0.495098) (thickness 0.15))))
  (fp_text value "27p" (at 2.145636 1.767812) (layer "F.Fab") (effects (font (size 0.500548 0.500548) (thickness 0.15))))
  (pad "1" smd roundrect (at -0.43 0 90) (size 0.6 0.54) (layers "F.Cu" "F.Paste" "F.Mask") (roundrect_rratio 0.14) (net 2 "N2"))
  (pad "2" smd roundrect (at 0.43 0 90) (size 0.6 0.54) (layers "F.Cu" "F.Paste" "F.Mask") (roundrect_rratio 0.14) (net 6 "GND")))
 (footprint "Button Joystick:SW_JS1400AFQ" (layer "F.Cu") (at 127.8 71.7)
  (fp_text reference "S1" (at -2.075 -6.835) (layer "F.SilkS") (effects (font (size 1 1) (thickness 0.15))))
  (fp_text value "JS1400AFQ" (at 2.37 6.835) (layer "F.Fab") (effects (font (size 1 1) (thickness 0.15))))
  (pad "" np_thru_hole circle (at 0 -1.9) (size 0.8 0.8) (drill 0.8) (layers "*.Cu" "*.Mask"))
  (pad "" np_thru_hole circle (at 0 1.9) (size 1.1 1.1) (drill 1.1) (layers "*.Cu" "*.Mask"))
  (pad "1" smd rect (at -4 -1.425) (size 2 1) (layers "F.Cu" "F.Paste" "F.Mask") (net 6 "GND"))
  (pad "2" smd rect (at -4 0) (size 2 1) (layers "F.Cu" "F.Paste" "F.Mask") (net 6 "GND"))
  (pad "3" smd rect (at -4 1.425) (size 2 1) (layers "F.Cu" "F.Paste" "F.Mask") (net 6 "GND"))
  (pad "4" smd rect (at 4 -1.425) (size 2 1) (layers "F.Cu" "F.Paste" "F.Mask") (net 39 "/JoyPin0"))
  (pad "5" smd rect (at 4 0) (size 2 1) (layers "F.Cu" "F.Paste" "F.Mask") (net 40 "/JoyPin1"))
  (pad "6" smd rect (at 4 1.425) (size 2 1) (layers "F.Cu" "F.Paste" "F.Mask") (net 41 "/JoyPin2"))
  (pad "G1" smd rect (at 0 -4.05) (size 2 1.8) (layers "F.Cu" "F.Paste" "F.Mask") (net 6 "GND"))
  (pad "G2" smd rect (at 0 4.05) (size 2 1.8) (layers "F.Cu" "F.Paste" "F.Mask") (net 6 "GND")))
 (gr_rect (start 118.2 64) (end 181.2 127) (stroke (width 1) (type solid)) (fill none) (layer "Edge.Cuts"))
 (segment (start 123.8 71.7) (end 123.8 73.125) (width 0.4) (layer "F.Cu") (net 6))
 (segment (start 125.175 70.275) (end 127.8 67.65) (width 0.4) (layer "F.Cu") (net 6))
 (segment (start 123.8 70.275) (end 125.175 70.275) (width 0.4) (layer "F.Cu") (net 6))
 (segment (start 123.8 70.275) (end 123.8 71.7) (width 0.4) (layer "F.Cu") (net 6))
 (segment (start 123.8 73.125) (end 125.175 73.125) (width 0.4) (layer "F.Cu") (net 6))
 (segment (start 125.175 73.125) (end 127.8 75.75) (width 0.4) (layer "F.Cu") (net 6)))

